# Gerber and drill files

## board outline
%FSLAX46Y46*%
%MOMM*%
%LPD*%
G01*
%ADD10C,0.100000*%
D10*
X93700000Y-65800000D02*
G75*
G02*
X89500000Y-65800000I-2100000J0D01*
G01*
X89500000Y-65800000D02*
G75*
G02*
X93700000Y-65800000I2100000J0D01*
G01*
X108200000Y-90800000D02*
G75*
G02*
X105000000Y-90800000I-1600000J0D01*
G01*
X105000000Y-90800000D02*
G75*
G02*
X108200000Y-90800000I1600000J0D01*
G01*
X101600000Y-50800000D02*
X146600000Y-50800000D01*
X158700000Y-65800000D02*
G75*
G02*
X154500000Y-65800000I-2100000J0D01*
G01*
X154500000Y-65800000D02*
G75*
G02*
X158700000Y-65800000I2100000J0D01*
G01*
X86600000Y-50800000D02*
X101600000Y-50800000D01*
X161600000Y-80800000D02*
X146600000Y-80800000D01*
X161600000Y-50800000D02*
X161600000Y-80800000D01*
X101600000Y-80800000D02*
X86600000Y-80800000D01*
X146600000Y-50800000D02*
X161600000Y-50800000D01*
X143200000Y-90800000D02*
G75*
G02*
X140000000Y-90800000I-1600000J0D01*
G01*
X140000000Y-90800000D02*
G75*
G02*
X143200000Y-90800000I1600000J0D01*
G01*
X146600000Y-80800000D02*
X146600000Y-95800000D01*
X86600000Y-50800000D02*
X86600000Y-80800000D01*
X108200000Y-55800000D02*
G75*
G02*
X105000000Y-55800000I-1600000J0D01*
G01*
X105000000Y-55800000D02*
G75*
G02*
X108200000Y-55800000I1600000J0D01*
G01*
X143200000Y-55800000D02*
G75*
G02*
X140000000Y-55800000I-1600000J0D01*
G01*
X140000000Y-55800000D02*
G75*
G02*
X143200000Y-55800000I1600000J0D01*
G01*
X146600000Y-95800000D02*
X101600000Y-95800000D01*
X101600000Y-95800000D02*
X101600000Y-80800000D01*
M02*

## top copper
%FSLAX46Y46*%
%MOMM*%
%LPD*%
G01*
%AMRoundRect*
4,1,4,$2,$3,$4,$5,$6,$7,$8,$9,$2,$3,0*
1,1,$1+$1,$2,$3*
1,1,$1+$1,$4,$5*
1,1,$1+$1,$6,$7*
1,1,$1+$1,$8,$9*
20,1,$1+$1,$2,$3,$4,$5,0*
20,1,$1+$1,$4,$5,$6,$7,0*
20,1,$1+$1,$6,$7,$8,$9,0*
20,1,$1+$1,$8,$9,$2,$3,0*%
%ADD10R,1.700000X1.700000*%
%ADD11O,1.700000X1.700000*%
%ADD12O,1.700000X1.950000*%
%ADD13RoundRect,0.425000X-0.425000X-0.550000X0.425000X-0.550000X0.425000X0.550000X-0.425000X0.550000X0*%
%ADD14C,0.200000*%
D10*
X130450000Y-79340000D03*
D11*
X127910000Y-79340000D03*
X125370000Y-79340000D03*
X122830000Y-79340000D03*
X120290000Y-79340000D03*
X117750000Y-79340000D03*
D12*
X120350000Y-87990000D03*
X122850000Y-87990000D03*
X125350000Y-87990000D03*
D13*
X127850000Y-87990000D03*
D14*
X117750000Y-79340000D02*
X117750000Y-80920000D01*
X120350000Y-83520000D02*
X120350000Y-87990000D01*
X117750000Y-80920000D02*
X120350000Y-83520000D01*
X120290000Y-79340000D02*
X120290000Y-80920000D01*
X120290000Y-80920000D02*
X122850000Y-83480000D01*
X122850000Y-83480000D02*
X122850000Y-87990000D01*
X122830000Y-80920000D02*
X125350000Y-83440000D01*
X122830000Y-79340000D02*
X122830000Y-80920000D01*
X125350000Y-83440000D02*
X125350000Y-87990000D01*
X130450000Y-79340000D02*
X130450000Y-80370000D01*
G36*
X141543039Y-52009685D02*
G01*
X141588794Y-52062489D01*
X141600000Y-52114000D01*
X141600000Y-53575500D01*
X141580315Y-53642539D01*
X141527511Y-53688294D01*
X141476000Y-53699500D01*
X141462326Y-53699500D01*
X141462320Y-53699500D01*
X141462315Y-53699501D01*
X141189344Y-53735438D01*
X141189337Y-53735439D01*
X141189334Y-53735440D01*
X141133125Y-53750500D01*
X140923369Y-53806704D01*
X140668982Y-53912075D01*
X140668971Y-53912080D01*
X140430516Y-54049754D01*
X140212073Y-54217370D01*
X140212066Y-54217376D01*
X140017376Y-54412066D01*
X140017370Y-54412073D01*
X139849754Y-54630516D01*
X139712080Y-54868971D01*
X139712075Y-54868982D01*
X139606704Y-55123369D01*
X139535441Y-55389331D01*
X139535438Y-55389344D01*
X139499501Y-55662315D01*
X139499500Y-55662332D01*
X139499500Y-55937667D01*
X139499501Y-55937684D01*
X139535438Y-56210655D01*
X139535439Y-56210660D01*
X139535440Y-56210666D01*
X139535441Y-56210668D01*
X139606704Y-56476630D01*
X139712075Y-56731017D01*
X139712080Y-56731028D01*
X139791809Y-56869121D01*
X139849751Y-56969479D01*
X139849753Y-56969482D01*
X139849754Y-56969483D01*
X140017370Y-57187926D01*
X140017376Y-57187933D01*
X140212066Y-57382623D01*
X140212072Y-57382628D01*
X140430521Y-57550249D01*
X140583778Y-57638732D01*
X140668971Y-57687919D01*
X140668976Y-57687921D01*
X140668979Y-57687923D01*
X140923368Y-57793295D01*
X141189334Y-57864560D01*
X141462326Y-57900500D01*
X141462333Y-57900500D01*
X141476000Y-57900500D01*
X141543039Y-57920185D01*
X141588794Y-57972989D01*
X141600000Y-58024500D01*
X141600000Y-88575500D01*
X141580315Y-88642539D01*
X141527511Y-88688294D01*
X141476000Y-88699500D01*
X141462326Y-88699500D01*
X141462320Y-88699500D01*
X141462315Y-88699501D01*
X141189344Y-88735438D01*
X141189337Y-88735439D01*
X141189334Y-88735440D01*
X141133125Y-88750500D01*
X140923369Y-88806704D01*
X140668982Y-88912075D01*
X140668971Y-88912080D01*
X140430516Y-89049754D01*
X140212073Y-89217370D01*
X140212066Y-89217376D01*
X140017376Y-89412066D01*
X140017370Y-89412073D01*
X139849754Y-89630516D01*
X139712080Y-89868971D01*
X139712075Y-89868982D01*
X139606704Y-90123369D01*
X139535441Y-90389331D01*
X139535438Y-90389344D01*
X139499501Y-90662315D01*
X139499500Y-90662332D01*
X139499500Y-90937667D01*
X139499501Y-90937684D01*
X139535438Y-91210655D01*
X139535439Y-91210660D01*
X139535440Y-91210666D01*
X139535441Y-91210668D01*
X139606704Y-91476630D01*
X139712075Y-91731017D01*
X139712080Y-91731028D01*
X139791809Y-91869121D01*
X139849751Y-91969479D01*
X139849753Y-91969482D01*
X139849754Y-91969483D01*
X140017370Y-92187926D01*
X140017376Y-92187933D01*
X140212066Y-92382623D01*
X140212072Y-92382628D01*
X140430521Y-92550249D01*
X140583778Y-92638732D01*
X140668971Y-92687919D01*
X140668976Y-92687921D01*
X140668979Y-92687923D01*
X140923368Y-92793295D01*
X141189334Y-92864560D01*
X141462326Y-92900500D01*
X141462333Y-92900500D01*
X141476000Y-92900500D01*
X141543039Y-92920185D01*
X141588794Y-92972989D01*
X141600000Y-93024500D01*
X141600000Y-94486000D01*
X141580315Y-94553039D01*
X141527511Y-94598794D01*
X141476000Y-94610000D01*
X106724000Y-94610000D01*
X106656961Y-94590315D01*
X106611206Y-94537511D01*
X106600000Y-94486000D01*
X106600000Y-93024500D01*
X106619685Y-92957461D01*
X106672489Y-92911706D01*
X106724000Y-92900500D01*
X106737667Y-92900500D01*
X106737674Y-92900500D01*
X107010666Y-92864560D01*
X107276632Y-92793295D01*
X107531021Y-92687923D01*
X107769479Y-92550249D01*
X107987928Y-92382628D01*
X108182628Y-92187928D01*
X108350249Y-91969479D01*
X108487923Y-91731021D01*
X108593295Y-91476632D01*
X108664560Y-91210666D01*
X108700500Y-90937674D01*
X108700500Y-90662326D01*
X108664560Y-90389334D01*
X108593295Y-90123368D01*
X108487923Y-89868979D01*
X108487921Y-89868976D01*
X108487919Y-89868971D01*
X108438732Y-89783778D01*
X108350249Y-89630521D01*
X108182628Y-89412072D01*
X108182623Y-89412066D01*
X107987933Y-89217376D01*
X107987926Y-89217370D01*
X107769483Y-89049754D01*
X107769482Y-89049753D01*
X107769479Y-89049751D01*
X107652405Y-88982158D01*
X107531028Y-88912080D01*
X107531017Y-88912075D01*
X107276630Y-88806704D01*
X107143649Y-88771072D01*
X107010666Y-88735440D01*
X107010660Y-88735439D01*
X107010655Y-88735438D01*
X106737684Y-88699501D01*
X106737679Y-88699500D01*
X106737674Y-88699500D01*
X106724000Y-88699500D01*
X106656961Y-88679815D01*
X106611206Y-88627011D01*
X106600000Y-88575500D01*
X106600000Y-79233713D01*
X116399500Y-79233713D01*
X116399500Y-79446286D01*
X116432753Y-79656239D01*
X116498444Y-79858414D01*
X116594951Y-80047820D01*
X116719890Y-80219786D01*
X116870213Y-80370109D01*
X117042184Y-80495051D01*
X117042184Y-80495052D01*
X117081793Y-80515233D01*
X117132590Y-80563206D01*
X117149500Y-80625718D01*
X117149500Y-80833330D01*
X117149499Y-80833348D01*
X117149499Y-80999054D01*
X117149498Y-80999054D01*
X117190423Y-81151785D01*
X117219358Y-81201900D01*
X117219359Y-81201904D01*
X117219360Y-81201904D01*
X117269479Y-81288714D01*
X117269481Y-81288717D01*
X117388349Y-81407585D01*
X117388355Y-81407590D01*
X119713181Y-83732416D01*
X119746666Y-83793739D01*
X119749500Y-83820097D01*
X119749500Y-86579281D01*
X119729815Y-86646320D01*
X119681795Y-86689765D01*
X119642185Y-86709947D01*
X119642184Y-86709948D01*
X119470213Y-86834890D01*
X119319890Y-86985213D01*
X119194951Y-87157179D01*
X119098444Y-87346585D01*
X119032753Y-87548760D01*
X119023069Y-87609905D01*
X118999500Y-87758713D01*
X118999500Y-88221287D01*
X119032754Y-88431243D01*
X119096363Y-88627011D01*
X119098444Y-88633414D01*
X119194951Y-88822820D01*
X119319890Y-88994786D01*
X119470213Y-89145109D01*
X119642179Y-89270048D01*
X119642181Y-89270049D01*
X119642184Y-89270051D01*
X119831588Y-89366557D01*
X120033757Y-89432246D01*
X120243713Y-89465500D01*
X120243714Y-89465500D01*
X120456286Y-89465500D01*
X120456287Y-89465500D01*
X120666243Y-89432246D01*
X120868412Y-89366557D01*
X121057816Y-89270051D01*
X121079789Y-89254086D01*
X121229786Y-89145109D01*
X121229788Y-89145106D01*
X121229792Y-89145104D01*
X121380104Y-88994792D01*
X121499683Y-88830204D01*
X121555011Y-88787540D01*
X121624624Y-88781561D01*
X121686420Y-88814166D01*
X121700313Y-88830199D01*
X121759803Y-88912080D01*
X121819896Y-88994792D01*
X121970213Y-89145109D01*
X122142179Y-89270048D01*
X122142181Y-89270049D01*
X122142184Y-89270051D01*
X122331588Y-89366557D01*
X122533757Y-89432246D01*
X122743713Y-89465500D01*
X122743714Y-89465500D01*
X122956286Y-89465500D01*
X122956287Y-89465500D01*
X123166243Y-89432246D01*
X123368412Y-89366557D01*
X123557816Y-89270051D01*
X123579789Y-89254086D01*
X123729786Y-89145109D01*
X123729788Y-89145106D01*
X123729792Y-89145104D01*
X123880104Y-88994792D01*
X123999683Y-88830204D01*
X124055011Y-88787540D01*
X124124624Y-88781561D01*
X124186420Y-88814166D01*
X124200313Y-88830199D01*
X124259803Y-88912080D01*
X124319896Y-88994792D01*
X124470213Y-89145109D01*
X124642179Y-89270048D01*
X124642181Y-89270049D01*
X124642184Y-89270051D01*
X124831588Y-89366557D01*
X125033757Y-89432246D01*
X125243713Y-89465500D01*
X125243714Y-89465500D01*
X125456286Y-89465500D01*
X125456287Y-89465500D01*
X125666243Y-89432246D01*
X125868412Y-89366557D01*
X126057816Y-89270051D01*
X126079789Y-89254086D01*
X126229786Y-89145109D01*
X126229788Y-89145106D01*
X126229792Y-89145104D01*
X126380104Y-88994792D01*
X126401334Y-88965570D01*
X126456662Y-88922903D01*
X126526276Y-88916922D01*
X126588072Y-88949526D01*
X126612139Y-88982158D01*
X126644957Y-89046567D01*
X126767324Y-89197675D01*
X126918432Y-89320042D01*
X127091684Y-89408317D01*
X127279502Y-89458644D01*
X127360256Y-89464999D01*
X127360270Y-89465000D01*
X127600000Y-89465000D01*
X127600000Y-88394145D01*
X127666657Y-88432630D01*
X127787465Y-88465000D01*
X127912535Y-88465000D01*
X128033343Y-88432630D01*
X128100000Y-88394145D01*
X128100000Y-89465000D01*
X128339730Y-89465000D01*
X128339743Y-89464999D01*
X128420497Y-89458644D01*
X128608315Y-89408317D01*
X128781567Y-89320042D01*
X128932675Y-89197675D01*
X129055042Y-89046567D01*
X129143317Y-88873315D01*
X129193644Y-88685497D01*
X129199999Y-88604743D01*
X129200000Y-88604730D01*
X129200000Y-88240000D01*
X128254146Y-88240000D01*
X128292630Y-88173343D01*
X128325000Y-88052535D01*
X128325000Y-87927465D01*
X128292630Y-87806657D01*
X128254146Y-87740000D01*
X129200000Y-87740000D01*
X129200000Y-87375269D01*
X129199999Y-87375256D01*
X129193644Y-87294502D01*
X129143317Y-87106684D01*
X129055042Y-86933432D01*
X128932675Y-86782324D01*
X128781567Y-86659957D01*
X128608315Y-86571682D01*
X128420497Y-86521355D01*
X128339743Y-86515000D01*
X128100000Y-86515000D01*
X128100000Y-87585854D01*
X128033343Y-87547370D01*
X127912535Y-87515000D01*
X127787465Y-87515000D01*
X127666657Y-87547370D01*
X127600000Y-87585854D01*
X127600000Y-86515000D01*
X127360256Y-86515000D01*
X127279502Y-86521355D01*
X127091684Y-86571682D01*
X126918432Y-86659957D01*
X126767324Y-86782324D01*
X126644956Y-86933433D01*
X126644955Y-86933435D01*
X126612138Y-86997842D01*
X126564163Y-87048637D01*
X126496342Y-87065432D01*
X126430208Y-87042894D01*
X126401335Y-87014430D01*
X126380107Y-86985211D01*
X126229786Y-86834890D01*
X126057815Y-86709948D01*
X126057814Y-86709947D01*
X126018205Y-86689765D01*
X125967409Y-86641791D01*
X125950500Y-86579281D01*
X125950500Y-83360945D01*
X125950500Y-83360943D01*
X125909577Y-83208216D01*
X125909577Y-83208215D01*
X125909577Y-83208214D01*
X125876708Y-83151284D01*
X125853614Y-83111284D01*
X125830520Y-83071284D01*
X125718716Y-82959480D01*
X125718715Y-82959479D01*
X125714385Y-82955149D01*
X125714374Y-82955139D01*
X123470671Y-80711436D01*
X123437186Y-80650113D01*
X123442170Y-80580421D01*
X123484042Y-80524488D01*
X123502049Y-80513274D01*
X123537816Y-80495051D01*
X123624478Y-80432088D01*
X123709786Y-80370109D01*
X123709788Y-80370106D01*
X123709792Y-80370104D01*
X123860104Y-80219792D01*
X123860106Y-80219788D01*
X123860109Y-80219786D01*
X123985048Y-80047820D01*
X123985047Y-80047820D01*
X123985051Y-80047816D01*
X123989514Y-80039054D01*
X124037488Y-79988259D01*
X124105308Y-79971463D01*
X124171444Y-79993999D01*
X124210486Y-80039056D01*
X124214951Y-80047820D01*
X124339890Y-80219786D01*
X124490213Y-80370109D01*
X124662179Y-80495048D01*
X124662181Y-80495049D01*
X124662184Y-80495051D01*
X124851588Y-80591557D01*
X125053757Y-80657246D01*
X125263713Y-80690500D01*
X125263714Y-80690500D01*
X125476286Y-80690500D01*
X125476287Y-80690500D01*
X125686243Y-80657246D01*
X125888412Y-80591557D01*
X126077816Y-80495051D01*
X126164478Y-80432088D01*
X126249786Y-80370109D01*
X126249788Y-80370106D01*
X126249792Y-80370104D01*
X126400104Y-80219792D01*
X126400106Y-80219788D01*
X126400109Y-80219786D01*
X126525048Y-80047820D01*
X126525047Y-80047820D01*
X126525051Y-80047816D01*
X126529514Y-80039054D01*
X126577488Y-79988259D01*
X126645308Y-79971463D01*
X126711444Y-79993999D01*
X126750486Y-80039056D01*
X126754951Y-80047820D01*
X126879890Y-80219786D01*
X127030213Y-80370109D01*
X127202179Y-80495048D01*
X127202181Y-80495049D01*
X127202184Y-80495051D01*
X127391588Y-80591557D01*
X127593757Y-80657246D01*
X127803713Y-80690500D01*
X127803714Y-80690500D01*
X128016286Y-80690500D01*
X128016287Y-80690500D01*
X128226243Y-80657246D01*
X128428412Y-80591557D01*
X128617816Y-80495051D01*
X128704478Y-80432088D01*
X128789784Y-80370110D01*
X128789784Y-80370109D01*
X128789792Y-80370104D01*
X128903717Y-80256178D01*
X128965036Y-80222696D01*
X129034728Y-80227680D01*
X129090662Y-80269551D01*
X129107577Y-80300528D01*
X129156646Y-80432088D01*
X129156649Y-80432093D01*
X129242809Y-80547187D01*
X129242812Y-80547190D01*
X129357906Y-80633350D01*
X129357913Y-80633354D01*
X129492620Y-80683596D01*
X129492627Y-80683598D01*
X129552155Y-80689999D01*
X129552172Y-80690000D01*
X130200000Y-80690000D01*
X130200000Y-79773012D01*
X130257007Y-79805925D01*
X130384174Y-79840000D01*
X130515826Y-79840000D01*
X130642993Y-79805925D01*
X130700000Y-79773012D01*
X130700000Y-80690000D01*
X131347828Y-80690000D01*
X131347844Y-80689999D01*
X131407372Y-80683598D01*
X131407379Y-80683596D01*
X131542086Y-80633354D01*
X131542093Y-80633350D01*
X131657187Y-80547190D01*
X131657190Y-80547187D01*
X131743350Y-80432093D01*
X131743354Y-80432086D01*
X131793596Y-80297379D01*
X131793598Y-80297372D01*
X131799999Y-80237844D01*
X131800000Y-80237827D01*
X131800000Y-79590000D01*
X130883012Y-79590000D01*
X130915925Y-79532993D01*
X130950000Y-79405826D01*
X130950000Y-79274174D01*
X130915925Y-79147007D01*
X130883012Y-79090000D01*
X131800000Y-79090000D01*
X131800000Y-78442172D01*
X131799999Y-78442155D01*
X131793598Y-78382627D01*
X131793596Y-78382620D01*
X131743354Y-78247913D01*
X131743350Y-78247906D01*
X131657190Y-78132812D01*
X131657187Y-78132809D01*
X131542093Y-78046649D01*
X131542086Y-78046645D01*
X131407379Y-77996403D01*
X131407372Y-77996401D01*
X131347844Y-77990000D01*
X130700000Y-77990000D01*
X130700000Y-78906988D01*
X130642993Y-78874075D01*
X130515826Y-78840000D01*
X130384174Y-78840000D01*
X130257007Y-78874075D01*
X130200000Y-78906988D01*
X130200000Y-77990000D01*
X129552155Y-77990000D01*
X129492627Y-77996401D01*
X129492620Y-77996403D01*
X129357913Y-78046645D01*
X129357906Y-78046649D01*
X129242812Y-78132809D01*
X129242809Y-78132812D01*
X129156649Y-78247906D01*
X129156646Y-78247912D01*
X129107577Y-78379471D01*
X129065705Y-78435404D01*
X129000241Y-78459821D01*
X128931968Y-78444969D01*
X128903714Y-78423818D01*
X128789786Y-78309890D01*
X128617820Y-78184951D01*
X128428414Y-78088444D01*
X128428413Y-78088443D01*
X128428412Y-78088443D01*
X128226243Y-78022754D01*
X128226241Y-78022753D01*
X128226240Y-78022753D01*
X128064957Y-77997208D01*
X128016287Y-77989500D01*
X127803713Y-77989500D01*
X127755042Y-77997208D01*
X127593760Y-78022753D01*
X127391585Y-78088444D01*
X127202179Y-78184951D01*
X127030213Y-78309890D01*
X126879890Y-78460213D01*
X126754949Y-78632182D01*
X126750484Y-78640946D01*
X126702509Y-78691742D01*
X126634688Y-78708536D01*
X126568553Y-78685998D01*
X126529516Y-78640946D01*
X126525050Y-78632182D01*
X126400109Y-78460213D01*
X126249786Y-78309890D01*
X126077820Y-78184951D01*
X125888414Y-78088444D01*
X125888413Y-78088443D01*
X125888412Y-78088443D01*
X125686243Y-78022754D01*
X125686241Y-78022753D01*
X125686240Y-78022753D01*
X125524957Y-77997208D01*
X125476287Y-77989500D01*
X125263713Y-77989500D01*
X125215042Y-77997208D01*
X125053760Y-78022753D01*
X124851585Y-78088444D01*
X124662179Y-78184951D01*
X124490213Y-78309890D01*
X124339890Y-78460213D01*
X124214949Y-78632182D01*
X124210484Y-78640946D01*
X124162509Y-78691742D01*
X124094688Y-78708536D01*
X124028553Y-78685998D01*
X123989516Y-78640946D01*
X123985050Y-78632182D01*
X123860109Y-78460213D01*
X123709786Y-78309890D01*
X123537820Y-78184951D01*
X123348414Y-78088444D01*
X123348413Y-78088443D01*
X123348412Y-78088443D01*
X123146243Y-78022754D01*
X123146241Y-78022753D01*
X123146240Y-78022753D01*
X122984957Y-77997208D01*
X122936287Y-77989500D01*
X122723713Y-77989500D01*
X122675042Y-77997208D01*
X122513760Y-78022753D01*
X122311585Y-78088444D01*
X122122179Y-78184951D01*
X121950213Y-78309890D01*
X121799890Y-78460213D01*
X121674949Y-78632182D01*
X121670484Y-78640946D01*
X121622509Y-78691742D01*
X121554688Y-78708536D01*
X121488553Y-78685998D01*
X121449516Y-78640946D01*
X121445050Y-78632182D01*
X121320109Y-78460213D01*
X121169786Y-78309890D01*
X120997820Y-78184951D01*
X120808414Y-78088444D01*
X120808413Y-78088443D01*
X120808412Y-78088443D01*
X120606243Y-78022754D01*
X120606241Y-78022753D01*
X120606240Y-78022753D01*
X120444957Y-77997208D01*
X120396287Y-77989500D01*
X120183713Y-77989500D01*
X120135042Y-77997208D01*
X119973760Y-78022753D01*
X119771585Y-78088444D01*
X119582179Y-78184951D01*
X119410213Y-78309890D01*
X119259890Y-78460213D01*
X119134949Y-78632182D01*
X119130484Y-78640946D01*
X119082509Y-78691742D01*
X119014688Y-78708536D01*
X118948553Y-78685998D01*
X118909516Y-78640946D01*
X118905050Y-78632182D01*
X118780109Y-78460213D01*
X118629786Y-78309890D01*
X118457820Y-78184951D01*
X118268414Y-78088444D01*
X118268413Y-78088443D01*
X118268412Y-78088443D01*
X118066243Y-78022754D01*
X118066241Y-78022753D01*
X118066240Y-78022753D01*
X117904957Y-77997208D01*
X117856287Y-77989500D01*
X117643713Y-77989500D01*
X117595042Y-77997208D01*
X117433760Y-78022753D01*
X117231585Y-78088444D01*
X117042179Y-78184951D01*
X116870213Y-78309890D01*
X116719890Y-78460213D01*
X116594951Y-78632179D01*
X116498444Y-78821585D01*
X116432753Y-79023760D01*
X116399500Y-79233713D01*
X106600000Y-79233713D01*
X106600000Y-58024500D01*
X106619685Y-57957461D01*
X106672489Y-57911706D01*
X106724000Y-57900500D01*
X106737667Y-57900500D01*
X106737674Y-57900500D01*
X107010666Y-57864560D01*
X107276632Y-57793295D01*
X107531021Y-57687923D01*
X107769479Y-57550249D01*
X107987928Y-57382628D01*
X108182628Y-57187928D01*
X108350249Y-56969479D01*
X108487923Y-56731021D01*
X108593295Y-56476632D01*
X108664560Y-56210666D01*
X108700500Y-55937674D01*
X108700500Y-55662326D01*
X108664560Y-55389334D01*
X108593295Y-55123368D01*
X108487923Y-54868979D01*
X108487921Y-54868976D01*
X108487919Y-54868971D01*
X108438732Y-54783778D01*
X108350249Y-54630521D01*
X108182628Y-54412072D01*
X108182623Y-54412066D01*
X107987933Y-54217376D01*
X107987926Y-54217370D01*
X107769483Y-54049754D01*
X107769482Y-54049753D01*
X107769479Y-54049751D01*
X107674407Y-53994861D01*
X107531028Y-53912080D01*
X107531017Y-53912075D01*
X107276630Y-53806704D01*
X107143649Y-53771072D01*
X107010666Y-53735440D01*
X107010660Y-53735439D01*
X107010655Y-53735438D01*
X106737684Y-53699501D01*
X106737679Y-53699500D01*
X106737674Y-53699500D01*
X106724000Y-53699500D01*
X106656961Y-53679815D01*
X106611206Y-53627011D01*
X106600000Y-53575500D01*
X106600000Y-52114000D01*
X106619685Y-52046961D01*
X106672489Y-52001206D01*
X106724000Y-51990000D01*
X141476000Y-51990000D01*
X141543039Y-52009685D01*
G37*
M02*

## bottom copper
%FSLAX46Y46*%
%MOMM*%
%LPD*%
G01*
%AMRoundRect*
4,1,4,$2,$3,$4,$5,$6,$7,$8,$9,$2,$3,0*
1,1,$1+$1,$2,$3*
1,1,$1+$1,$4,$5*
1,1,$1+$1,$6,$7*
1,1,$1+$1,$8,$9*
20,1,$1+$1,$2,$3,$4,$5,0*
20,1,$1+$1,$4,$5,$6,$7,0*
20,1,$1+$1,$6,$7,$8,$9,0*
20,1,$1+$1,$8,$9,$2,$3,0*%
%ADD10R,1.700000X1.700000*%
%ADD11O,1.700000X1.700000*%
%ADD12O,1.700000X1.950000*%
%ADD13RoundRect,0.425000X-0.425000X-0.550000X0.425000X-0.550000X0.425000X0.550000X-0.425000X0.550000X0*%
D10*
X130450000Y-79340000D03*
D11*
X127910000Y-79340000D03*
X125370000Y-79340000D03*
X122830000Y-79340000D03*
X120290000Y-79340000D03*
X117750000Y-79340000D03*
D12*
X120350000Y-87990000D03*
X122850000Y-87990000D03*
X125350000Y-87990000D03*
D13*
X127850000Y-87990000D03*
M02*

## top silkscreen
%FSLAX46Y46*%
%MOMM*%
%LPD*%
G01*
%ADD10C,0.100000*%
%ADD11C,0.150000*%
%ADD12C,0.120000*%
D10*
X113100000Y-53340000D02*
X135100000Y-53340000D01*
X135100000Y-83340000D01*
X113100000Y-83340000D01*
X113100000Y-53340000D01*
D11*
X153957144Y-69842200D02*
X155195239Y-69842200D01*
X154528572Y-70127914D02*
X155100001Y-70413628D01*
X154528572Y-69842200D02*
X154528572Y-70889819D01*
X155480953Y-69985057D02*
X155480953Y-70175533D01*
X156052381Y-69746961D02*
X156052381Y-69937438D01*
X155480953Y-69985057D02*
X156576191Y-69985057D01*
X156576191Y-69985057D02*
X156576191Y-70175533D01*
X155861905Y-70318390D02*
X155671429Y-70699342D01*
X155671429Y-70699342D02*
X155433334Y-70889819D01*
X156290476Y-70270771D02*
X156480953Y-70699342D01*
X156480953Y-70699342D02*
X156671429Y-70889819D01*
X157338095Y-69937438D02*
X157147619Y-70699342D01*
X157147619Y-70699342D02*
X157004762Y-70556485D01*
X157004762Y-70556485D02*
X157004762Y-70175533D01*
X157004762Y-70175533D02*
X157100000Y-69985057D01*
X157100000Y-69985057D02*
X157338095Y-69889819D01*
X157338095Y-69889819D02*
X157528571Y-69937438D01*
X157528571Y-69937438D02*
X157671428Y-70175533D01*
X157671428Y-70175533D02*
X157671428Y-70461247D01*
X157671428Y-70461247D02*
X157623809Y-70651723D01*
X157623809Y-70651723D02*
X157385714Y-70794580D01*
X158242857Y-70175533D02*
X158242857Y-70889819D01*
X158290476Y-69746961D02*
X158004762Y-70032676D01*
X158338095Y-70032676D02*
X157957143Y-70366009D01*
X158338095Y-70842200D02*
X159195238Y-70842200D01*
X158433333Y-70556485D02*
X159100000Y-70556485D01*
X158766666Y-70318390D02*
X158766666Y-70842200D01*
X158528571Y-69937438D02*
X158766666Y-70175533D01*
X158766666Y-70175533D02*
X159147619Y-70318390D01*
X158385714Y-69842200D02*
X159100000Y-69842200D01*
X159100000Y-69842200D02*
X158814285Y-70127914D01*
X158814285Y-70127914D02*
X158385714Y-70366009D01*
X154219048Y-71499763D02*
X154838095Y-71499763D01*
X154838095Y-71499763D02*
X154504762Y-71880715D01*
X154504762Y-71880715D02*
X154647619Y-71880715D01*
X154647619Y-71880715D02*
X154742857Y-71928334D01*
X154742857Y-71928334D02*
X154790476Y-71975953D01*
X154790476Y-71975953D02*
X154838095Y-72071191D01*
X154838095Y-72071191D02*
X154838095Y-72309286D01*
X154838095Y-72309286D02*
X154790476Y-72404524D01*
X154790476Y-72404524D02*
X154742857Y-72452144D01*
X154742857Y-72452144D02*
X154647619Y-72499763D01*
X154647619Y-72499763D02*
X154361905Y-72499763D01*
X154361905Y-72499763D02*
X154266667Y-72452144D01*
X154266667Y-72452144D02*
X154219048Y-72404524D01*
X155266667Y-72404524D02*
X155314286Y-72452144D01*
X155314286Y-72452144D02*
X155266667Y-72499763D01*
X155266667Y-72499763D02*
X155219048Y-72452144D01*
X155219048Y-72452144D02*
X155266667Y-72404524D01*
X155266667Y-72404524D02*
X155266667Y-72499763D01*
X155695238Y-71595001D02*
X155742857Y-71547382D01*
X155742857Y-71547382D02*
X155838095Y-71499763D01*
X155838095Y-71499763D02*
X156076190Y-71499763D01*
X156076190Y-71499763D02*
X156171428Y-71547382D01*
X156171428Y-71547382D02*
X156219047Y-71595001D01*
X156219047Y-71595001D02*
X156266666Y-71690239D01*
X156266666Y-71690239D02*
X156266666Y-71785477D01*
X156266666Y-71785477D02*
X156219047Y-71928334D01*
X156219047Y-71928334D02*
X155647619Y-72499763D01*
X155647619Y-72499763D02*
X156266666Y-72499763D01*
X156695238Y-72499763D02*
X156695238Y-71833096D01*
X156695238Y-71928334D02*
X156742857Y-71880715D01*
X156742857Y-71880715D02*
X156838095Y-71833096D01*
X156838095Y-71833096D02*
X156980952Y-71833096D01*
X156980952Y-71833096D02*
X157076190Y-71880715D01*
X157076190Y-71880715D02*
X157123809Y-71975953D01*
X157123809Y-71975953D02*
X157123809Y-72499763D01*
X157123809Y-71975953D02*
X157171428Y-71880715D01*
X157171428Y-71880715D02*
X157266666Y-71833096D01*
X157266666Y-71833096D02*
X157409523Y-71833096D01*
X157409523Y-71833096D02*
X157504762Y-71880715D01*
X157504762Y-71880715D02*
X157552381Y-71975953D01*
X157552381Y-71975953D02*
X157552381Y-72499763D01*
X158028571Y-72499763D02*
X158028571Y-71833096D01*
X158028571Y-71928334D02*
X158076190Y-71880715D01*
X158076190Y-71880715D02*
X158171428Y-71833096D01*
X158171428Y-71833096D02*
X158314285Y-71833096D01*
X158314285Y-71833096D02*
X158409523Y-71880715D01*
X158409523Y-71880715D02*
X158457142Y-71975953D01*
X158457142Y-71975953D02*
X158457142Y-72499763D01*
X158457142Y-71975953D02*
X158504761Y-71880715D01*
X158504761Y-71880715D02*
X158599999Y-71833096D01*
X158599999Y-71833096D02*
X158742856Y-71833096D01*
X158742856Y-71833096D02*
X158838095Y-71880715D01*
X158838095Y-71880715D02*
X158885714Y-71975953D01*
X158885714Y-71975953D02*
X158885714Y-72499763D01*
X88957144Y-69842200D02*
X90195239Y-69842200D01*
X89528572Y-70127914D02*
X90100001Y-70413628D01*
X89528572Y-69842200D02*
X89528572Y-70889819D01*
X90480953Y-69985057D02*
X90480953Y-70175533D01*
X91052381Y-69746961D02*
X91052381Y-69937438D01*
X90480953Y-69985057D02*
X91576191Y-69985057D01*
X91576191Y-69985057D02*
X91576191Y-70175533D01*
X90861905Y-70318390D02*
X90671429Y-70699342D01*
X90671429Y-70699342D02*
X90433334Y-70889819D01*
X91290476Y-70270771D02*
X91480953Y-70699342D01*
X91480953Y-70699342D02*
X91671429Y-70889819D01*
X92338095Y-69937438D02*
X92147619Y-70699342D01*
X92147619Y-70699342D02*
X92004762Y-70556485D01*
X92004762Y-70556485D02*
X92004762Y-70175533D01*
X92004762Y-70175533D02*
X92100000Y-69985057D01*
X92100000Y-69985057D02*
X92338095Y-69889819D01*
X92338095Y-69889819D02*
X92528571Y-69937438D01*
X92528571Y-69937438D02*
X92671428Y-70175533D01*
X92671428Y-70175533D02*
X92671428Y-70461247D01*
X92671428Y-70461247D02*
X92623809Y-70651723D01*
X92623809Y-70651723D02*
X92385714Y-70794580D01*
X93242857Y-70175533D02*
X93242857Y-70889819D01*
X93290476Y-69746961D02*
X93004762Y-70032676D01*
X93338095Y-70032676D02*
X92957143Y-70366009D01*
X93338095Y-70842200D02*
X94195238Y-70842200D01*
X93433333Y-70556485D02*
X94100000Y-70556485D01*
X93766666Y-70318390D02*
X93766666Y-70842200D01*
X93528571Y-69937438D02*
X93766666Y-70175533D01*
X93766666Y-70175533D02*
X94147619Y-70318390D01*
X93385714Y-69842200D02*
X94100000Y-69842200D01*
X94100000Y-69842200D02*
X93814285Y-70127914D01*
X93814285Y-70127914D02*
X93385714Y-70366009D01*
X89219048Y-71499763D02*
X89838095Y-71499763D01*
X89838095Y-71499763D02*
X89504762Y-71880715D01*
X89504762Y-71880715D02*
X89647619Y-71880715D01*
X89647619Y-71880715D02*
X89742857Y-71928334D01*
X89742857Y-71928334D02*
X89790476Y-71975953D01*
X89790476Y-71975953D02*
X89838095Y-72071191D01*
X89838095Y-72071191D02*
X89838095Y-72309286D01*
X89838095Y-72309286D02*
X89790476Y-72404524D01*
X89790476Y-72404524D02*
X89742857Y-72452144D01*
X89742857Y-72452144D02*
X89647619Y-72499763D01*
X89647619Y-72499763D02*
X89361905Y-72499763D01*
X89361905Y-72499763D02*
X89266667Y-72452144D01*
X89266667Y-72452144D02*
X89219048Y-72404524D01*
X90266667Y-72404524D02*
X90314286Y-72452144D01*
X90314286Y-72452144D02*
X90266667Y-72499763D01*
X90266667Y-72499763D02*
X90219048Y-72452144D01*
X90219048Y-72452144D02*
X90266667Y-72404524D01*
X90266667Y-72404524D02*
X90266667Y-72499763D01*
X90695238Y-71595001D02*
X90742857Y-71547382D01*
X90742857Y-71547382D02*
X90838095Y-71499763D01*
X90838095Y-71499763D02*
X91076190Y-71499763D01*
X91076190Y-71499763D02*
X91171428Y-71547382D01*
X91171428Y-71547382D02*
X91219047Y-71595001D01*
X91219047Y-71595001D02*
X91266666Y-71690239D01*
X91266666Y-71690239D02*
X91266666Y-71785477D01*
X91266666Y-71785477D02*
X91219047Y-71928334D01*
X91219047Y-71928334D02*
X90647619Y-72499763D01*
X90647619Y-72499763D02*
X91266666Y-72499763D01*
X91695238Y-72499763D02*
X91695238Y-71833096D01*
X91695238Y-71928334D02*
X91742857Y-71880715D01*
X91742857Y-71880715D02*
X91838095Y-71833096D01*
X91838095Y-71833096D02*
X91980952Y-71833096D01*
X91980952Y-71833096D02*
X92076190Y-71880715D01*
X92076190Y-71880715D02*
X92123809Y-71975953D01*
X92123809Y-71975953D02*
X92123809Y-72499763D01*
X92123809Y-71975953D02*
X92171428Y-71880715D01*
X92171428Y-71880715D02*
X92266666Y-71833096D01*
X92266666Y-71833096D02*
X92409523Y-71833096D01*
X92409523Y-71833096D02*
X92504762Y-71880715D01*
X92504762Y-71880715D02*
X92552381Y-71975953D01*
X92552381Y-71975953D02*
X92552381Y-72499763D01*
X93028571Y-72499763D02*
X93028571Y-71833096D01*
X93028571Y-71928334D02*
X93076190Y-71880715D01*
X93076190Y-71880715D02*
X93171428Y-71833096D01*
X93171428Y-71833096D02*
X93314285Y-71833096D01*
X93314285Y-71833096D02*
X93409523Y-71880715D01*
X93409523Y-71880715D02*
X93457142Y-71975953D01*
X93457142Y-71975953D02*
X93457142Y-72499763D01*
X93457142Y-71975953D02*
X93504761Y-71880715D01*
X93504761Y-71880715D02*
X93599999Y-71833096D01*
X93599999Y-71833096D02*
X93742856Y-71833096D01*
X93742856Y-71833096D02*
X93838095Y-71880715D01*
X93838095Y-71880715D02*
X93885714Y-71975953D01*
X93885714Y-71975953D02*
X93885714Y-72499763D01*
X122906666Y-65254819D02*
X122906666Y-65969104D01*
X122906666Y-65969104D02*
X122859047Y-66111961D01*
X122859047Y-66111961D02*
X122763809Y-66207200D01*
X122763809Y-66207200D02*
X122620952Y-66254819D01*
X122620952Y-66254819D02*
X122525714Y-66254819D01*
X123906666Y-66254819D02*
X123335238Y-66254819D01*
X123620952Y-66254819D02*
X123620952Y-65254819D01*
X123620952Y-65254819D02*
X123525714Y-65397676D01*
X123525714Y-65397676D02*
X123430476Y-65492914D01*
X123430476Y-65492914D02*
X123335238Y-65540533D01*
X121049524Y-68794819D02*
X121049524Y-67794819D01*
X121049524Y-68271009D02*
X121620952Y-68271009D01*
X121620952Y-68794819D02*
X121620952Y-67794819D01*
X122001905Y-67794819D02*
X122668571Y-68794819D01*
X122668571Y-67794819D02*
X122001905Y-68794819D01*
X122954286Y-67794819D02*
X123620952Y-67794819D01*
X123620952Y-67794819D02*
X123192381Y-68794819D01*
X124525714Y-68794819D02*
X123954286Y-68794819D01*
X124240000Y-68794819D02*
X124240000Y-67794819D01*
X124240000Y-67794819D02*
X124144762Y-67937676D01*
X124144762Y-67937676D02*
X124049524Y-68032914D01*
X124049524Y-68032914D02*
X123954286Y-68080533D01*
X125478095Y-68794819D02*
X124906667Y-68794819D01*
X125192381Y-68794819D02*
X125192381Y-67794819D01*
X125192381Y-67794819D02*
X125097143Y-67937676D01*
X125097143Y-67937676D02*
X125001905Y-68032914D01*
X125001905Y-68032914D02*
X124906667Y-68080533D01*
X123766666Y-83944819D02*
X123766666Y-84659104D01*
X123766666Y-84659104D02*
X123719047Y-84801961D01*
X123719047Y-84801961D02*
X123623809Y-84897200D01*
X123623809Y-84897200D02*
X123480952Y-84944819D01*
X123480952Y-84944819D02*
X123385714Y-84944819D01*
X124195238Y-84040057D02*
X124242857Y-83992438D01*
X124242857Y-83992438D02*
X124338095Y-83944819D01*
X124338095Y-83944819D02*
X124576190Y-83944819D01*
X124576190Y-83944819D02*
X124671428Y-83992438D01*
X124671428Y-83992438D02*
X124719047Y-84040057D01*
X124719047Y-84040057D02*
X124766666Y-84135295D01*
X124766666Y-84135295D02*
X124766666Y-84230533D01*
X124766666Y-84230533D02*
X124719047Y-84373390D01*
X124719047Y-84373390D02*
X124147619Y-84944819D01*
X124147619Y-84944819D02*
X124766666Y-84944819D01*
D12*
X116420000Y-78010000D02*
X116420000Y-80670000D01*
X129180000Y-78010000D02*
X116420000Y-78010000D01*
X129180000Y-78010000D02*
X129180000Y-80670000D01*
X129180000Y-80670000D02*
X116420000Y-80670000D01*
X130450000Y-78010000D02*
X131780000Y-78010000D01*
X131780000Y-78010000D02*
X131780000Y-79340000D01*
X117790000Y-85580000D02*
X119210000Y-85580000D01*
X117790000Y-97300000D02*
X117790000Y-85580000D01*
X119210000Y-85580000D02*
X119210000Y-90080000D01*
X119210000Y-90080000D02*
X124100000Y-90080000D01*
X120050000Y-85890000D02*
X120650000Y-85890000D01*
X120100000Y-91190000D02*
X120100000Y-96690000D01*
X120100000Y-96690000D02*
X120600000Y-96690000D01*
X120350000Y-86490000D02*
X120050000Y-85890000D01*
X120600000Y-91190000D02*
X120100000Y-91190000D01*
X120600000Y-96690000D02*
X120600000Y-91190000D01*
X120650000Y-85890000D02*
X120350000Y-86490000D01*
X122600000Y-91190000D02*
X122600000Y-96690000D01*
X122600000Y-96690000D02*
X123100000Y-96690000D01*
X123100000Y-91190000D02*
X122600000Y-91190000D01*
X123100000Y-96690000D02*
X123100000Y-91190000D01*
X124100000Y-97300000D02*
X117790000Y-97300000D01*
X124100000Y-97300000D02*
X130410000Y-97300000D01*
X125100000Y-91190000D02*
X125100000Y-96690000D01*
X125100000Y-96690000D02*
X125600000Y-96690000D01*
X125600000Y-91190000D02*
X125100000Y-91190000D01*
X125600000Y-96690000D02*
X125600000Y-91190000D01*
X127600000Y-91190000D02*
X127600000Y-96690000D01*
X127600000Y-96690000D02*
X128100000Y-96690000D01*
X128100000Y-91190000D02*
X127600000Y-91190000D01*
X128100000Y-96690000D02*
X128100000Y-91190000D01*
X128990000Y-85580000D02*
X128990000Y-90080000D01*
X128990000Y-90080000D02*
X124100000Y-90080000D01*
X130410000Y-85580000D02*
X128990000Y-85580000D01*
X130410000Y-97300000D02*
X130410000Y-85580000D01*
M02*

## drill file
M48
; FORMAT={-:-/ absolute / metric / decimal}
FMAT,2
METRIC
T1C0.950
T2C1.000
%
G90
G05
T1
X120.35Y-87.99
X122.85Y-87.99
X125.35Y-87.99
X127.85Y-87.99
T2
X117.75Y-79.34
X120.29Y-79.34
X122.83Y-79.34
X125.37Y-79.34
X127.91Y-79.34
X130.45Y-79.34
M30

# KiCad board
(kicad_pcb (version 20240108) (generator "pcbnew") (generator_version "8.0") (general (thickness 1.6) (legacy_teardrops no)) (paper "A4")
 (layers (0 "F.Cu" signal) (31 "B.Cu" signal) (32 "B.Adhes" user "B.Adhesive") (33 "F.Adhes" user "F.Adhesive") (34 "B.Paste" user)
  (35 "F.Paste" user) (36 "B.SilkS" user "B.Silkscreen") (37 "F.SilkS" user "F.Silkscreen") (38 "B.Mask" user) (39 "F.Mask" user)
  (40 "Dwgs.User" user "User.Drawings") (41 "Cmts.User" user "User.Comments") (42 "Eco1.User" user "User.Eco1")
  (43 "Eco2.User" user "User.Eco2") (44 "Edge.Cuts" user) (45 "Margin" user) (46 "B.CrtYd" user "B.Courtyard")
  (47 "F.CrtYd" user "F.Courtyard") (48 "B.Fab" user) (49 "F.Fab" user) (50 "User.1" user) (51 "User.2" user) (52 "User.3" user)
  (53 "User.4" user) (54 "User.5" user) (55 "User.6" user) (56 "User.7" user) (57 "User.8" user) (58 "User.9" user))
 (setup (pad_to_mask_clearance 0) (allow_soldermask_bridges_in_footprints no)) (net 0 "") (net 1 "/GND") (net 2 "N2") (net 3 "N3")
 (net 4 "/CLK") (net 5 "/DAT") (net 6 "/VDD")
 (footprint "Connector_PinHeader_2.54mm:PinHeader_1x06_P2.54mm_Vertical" (layer "F.Cu") (at 130.45 79.34 -90)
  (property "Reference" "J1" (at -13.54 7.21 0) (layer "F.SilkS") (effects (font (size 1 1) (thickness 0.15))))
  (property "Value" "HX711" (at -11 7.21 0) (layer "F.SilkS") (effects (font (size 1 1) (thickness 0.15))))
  (fp_line (start -1.33 14.03) (end 1.33 14.03) (stroke (width 0.12) (type solid)) (layer "F.SilkS"))
  (fp_line (start -1.33 1.27) (end -1.33 14.03) (stroke (width 0.12) (type solid)) (layer "F.SilkS"))
  (fp_line (start -1.33 1.27) (end 1.33 1.27) (stroke (width 0.12) (type solid)) (layer "F.SilkS"))
  (fp_line (start 1.33 1.27) (end 1.33 14.03) (stroke (width 0.12) (type solid)) (layer "F.SilkS"))
  (fp_line (start -1.33 0) (end -1.33 -1.33) (stroke (width 0.12) (type solid)) (layer "F.SilkS"))
  (fp_line (start -1.33 -1.33) (end 0 -1.33) (stroke (width 0.12) (type solid)) (layer "F.SilkS"))
  (pad "1" thru_hole rect (at 0 0 270) (size 1.7 1.7) (drill 1) (layers "*.Cu" "*.Mask") (remove_unused_layers no) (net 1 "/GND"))
  (pad "2" thru_hole oval (at 0 2.54 270) (size 1.7 1.7) (drill 1) (layers "*.Cu" "*.Mask") (remove_unused_layers no) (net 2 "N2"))
  (pad "3" thru_hole oval (at 0 5.08 270) (size 1.7 1.7) (drill 1) (layers "*.Cu" "*.Mask") (remove_unused_layers no) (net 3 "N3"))
  (pad "4" thru_hole oval (at 0 7.62 270) (size 1.7 1.7) (drill 1) (layers "*.Cu" "*.Mask") (remove_unused_layers no) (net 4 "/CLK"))
  (pad "5" thru_hole oval (at 0 10.16 270) (size 1.7 1.7) (drill 1) (layers "*.Cu" "*.Mask") (remove_unused_layers no) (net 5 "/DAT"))
  (pad "6" thru_hole oval (at 0 12.7 270) (size 1.7 1.7) (drill 1) (layers "*.Cu" "*.Mask") (remove_unused_layers no) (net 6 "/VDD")))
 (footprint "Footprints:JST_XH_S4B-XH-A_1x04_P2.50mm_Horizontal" (layer "F.Cu") (at 120.35 87.99)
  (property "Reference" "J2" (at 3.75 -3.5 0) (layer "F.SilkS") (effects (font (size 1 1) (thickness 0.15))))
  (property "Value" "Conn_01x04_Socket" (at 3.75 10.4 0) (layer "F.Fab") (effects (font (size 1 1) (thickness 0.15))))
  (fp_line (start -2.56 -2.41) (end -1.14 -2.41) (stroke (width 0.12) (type solid)) (layer "F.SilkS"))
  (fp_line (start -2.56 9.31) (end -2.56 -2.41) (stroke (width 0.12) (type solid)) (layer "F.SilkS"))
  (fp_line (start -1.14 -2.41) (end -1.14 2.09) (stroke (width 0.12) (type solid)) (layer "F.SilkS"))
  (fp_line (start -1.14 2.09) (end 3.75 2.09) (stroke (width 0.12) (type solid)) (layer "F.SilkS"))
  (fp_line (start -0.3 -2.1) (end 0.3 -2.1) (stroke (width 0.12) (type solid)) (layer "F.SilkS"))
  (fp_line (start -0.25 3.2) (end -0.25 8.7) (stroke (width 0.12) (type solid)) (layer "F.SilkS"))
  (fp_line (start -0.25 8.7) (end 0.25 8.7) (stroke (width 0.12) (type solid)) (layer "F.SilkS"))
  (fp_line (start 0 -1.5) (end -0.3 -2.1) (stroke (width 0.12) (type solid)) (layer "F.SilkS"))
  (fp_line (start 0.25 3.2) (end -0.25 3.2) (stroke (width 0.12) (type solid)) (layer "F.SilkS"))
  (fp_line (start 0.25 8.7) (end 0.25 3.2) (stroke (width 0.12) (type solid)) (layer "F.SilkS"))
  (fp_line (start 0.3 -2.1) (end 0 -1.5) (stroke (width 0.12) (type solid)) (layer "F.SilkS"))
  (fp_line (start 2.25 3.2) (end 2.25 8.7) (stroke (width 0.12) (type solid)) (layer "F.SilkS"))
  (fp_line (start 2.25 8.7) (end 2.75 8.7) (stroke (width 0.12) (type solid)) (layer "F.SilkS"))
  (fp_line (start 2.75 3.2) (end 2.25 3.2) (stroke (width 0.12) (type solid)) (layer "F.SilkS"))
  (fp_line (start 2.75 8.7) (end 2.75 3.2) (stroke (width 0.12) (type solid)) (layer "F.SilkS"))
  (fp_line (start 3.75 9.31) (end -2.56 9.31) (stroke (width 0.12) (type solid)) (layer "F.SilkS"))
  (fp_line (start 3.75 9.31) (end 10.06 9.31) (stroke (width 0.12) (type solid)) (layer "F.SilkS"))
  (fp_line (start 4.75 3.2) (end 4.75 8.7) (stroke (width 0.12) (type solid)) (layer "F.SilkS"))
  (fp_line (start 4.75 8.7) (end 5.25 8.7) (stroke (width 0.12) (type solid)) (layer "F.SilkS"))
  (fp_line (start 5.25 3.2) (end 4.75 3.2) (stroke (width 0.12) (type solid)) (layer "F.SilkS"))
  (fp_line (start 5.25 8.7) (end 5.25 3.2) (stroke (width 0.12) (type solid)) (layer "F.SilkS"))
  (fp_line (start 7.25 3.2) (end 7.25 8.7) (stroke (width 0.12) (type solid)) (layer "F.SilkS"))
  (fp_line (start 7.25 8.7) (end 7.75 8.7) (stroke (width 0.12) (type solid)) (layer "F.SilkS"))
  (fp_line (start 7.75 3.2) (end 7.25 3.2) (stroke (width 0.12) (type solid)) (layer "F.SilkS"))
  (fp_line (start 7.75 8.7) (end 7.75 3.2) (stroke (width 0.12) (type solid)) (layer "F.SilkS"))
  (fp_line (start 8.64 -2.41) (end 8.64 2.09) (stroke (width 0.12) (type solid)) (layer "F.SilkS"))
  (fp_line (start 8.64 2.09) (end 3.75 2.09) (stroke (width 0.12) (type solid)) (layer "F.SilkS"))
  (fp_line (start 10.06 -2.41) (end 8.64 -2.41) (stroke (width 0.12) (type solid)) (layer "F.SilkS"))
  (fp_line (start 10.06 9.31) (end 10.06 -2.41) (stroke (width 0.12) (type solid)) (layer "F.SilkS"))
  (pad "1" thru_hole oval (at 0 0) (size 1.7 1.95) (drill 0.95) (layers "*.Cu" "*.Mask") (remove_unused_layers no) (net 6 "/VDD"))
  (pad "2" thru_hole oval (at 2.5 0) (size 1.7 1.95) (drill 0.95) (layers "*.Cu" "*.Mask") (remove_unused_layers no) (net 5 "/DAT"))
  (pad "3" thru_hole oval (at 5 0) (size 1.7 1.95) (drill 0.95) (layers "*.Cu" "*.Mask") (remove_unused_layers no) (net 4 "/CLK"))
  (pad "4" thru_hole roundrect (at 7.5 0) (size 1.7 1.95) (drill 0.95) (layers "*.Cu" "*.Mask") (remove_unused_layers no)
   (roundrect_rratio 0.25) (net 1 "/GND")))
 (gr_rect (start 113.1 53.34) (end 135.1 83.34) (stroke (width 0.1) (type default)) (fill none) (layer "F.SilkS"))
 (gr_circle (center 91.6 65.8) (end 93.7 65.8) (stroke (width 0.1) (type default)) (fill none) (layer "Edge.Cuts"))
 (gr_circle (center 106.6 90.8) (end 108.2 90.8) (stroke (width 0.1) (type default)) (fill none) (layer "Edge.Cuts"))
 (gr_line (start 101.6 50.8) (end 146.6 50.8) (stroke (width 0.1) (type default)) (layer "Edge.Cuts"))
 (gr_circle (center 156.6 65.8) (end 158.7 65.8) (stroke (width 0.1) (type default)) (fill none) (layer "Edge.Cuts"))
 (gr_line (start 86.6 50.8) (end 101.6 50.8) (stroke (width 0.1) (type default)) (layer "Edge.Cuts"))
 (gr_line (start 161.6 80.8) (end 146.6 80.8) (stroke (width 0.1) (type default)) (layer "Edge.Cuts"))
 (gr_line (start 161.6 50.8) (end 161.6 80.8) (stroke (width 0.1) (type default)) (layer "Edge.Cuts"))
 (gr_line (start 101.6 80.8) (end 86.6 80.8) (stroke (width 0.1) (type default)) (layer "Edge.Cuts"))
 (gr_line (start 146.6 50.8) (end 161.6 50.8) (stroke (width 0.1) (type default)) (layer "Edge.Cuts"))
 (gr_circle (center 141.6 90.8) (end 143.2 90.8) (stroke (width 0.1) (type default)) (fill none) (layer "Edge.Cuts"))
 (gr_line (start 146.6 80.8) (end 146.6 95.8) (stroke (width 0.1) (type default)) (layer "Edge.Cuts"))
 (gr_line (start 86.6 50.8) (end 86.6 80.8) (stroke (width 0.1) (type default)) (layer "Edge.Cuts"))
 (gr_circle (center 106.6 55.8) (end 108.2 55.8) (stroke (width 0.1) (type default)) (fill none) (layer "Edge.Cuts"))
 (gr_circle (center 141.6 55.8) (end 143.2 55.8) (stroke (width 0.1) (type default)) (fill none) (layer "Edge.Cuts"))
 (gr_line (start 146.6 95.8) (end 101.6 95.8) (stroke (width 0.1) (type default)) (layer "Edge.Cuts"))
 (gr_line (start 101.6 95.8) (end 101.6 80.8) (stroke (width 0.1) (type default)) (layer "Edge.Cuts"))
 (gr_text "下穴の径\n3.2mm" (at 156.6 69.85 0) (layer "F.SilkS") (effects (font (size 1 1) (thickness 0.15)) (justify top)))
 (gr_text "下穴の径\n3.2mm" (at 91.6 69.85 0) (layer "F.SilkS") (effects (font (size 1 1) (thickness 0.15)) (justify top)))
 (segment (start 117.75 79.34) (end 117.75 80.92) (width 0.2) (layer "F.Cu") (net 6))
 (segment (start 120.35 83.52) (end 120.35 87.99) (width 0.2) (layer "F.Cu") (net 6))
 (segment (start 117.75 80.92) (end 120.35 83.52) (width 0.2) (layer "F.Cu") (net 6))
 (segment (start 120.29 79.34) (end 120.29 80.92) (width 0.2) (layer "F.Cu") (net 5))
 (segment (start 120.29 80.92) (end 122.85 83.48) (width 0.2) (layer "F.Cu") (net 5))
 (segment (start 122.85 83.48) (end 122.85 87.99) (width 0.2) (layer "F.Cu") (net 5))
 (segment (start 122.83 80.92) (end 125.35 83.44) (width 0.2) (layer "F.Cu") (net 4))
 (segment (start 122.83 79.34) (end 122.83 80.92) (width 0.2) (layer "F.Cu") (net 4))
 (segment (start 125.35 83.44) (end 125.35 87.99) (width 0.2) (layer "F.Cu") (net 4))
 (segment (start 130.45 79.34) (end 130.45 80.37) (width 0.2) (layer "F.Cu") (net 1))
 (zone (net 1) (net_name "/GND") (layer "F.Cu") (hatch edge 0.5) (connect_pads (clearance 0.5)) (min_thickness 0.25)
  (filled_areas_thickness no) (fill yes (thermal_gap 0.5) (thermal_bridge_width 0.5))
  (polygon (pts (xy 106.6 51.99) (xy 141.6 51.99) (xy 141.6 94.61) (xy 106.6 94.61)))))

